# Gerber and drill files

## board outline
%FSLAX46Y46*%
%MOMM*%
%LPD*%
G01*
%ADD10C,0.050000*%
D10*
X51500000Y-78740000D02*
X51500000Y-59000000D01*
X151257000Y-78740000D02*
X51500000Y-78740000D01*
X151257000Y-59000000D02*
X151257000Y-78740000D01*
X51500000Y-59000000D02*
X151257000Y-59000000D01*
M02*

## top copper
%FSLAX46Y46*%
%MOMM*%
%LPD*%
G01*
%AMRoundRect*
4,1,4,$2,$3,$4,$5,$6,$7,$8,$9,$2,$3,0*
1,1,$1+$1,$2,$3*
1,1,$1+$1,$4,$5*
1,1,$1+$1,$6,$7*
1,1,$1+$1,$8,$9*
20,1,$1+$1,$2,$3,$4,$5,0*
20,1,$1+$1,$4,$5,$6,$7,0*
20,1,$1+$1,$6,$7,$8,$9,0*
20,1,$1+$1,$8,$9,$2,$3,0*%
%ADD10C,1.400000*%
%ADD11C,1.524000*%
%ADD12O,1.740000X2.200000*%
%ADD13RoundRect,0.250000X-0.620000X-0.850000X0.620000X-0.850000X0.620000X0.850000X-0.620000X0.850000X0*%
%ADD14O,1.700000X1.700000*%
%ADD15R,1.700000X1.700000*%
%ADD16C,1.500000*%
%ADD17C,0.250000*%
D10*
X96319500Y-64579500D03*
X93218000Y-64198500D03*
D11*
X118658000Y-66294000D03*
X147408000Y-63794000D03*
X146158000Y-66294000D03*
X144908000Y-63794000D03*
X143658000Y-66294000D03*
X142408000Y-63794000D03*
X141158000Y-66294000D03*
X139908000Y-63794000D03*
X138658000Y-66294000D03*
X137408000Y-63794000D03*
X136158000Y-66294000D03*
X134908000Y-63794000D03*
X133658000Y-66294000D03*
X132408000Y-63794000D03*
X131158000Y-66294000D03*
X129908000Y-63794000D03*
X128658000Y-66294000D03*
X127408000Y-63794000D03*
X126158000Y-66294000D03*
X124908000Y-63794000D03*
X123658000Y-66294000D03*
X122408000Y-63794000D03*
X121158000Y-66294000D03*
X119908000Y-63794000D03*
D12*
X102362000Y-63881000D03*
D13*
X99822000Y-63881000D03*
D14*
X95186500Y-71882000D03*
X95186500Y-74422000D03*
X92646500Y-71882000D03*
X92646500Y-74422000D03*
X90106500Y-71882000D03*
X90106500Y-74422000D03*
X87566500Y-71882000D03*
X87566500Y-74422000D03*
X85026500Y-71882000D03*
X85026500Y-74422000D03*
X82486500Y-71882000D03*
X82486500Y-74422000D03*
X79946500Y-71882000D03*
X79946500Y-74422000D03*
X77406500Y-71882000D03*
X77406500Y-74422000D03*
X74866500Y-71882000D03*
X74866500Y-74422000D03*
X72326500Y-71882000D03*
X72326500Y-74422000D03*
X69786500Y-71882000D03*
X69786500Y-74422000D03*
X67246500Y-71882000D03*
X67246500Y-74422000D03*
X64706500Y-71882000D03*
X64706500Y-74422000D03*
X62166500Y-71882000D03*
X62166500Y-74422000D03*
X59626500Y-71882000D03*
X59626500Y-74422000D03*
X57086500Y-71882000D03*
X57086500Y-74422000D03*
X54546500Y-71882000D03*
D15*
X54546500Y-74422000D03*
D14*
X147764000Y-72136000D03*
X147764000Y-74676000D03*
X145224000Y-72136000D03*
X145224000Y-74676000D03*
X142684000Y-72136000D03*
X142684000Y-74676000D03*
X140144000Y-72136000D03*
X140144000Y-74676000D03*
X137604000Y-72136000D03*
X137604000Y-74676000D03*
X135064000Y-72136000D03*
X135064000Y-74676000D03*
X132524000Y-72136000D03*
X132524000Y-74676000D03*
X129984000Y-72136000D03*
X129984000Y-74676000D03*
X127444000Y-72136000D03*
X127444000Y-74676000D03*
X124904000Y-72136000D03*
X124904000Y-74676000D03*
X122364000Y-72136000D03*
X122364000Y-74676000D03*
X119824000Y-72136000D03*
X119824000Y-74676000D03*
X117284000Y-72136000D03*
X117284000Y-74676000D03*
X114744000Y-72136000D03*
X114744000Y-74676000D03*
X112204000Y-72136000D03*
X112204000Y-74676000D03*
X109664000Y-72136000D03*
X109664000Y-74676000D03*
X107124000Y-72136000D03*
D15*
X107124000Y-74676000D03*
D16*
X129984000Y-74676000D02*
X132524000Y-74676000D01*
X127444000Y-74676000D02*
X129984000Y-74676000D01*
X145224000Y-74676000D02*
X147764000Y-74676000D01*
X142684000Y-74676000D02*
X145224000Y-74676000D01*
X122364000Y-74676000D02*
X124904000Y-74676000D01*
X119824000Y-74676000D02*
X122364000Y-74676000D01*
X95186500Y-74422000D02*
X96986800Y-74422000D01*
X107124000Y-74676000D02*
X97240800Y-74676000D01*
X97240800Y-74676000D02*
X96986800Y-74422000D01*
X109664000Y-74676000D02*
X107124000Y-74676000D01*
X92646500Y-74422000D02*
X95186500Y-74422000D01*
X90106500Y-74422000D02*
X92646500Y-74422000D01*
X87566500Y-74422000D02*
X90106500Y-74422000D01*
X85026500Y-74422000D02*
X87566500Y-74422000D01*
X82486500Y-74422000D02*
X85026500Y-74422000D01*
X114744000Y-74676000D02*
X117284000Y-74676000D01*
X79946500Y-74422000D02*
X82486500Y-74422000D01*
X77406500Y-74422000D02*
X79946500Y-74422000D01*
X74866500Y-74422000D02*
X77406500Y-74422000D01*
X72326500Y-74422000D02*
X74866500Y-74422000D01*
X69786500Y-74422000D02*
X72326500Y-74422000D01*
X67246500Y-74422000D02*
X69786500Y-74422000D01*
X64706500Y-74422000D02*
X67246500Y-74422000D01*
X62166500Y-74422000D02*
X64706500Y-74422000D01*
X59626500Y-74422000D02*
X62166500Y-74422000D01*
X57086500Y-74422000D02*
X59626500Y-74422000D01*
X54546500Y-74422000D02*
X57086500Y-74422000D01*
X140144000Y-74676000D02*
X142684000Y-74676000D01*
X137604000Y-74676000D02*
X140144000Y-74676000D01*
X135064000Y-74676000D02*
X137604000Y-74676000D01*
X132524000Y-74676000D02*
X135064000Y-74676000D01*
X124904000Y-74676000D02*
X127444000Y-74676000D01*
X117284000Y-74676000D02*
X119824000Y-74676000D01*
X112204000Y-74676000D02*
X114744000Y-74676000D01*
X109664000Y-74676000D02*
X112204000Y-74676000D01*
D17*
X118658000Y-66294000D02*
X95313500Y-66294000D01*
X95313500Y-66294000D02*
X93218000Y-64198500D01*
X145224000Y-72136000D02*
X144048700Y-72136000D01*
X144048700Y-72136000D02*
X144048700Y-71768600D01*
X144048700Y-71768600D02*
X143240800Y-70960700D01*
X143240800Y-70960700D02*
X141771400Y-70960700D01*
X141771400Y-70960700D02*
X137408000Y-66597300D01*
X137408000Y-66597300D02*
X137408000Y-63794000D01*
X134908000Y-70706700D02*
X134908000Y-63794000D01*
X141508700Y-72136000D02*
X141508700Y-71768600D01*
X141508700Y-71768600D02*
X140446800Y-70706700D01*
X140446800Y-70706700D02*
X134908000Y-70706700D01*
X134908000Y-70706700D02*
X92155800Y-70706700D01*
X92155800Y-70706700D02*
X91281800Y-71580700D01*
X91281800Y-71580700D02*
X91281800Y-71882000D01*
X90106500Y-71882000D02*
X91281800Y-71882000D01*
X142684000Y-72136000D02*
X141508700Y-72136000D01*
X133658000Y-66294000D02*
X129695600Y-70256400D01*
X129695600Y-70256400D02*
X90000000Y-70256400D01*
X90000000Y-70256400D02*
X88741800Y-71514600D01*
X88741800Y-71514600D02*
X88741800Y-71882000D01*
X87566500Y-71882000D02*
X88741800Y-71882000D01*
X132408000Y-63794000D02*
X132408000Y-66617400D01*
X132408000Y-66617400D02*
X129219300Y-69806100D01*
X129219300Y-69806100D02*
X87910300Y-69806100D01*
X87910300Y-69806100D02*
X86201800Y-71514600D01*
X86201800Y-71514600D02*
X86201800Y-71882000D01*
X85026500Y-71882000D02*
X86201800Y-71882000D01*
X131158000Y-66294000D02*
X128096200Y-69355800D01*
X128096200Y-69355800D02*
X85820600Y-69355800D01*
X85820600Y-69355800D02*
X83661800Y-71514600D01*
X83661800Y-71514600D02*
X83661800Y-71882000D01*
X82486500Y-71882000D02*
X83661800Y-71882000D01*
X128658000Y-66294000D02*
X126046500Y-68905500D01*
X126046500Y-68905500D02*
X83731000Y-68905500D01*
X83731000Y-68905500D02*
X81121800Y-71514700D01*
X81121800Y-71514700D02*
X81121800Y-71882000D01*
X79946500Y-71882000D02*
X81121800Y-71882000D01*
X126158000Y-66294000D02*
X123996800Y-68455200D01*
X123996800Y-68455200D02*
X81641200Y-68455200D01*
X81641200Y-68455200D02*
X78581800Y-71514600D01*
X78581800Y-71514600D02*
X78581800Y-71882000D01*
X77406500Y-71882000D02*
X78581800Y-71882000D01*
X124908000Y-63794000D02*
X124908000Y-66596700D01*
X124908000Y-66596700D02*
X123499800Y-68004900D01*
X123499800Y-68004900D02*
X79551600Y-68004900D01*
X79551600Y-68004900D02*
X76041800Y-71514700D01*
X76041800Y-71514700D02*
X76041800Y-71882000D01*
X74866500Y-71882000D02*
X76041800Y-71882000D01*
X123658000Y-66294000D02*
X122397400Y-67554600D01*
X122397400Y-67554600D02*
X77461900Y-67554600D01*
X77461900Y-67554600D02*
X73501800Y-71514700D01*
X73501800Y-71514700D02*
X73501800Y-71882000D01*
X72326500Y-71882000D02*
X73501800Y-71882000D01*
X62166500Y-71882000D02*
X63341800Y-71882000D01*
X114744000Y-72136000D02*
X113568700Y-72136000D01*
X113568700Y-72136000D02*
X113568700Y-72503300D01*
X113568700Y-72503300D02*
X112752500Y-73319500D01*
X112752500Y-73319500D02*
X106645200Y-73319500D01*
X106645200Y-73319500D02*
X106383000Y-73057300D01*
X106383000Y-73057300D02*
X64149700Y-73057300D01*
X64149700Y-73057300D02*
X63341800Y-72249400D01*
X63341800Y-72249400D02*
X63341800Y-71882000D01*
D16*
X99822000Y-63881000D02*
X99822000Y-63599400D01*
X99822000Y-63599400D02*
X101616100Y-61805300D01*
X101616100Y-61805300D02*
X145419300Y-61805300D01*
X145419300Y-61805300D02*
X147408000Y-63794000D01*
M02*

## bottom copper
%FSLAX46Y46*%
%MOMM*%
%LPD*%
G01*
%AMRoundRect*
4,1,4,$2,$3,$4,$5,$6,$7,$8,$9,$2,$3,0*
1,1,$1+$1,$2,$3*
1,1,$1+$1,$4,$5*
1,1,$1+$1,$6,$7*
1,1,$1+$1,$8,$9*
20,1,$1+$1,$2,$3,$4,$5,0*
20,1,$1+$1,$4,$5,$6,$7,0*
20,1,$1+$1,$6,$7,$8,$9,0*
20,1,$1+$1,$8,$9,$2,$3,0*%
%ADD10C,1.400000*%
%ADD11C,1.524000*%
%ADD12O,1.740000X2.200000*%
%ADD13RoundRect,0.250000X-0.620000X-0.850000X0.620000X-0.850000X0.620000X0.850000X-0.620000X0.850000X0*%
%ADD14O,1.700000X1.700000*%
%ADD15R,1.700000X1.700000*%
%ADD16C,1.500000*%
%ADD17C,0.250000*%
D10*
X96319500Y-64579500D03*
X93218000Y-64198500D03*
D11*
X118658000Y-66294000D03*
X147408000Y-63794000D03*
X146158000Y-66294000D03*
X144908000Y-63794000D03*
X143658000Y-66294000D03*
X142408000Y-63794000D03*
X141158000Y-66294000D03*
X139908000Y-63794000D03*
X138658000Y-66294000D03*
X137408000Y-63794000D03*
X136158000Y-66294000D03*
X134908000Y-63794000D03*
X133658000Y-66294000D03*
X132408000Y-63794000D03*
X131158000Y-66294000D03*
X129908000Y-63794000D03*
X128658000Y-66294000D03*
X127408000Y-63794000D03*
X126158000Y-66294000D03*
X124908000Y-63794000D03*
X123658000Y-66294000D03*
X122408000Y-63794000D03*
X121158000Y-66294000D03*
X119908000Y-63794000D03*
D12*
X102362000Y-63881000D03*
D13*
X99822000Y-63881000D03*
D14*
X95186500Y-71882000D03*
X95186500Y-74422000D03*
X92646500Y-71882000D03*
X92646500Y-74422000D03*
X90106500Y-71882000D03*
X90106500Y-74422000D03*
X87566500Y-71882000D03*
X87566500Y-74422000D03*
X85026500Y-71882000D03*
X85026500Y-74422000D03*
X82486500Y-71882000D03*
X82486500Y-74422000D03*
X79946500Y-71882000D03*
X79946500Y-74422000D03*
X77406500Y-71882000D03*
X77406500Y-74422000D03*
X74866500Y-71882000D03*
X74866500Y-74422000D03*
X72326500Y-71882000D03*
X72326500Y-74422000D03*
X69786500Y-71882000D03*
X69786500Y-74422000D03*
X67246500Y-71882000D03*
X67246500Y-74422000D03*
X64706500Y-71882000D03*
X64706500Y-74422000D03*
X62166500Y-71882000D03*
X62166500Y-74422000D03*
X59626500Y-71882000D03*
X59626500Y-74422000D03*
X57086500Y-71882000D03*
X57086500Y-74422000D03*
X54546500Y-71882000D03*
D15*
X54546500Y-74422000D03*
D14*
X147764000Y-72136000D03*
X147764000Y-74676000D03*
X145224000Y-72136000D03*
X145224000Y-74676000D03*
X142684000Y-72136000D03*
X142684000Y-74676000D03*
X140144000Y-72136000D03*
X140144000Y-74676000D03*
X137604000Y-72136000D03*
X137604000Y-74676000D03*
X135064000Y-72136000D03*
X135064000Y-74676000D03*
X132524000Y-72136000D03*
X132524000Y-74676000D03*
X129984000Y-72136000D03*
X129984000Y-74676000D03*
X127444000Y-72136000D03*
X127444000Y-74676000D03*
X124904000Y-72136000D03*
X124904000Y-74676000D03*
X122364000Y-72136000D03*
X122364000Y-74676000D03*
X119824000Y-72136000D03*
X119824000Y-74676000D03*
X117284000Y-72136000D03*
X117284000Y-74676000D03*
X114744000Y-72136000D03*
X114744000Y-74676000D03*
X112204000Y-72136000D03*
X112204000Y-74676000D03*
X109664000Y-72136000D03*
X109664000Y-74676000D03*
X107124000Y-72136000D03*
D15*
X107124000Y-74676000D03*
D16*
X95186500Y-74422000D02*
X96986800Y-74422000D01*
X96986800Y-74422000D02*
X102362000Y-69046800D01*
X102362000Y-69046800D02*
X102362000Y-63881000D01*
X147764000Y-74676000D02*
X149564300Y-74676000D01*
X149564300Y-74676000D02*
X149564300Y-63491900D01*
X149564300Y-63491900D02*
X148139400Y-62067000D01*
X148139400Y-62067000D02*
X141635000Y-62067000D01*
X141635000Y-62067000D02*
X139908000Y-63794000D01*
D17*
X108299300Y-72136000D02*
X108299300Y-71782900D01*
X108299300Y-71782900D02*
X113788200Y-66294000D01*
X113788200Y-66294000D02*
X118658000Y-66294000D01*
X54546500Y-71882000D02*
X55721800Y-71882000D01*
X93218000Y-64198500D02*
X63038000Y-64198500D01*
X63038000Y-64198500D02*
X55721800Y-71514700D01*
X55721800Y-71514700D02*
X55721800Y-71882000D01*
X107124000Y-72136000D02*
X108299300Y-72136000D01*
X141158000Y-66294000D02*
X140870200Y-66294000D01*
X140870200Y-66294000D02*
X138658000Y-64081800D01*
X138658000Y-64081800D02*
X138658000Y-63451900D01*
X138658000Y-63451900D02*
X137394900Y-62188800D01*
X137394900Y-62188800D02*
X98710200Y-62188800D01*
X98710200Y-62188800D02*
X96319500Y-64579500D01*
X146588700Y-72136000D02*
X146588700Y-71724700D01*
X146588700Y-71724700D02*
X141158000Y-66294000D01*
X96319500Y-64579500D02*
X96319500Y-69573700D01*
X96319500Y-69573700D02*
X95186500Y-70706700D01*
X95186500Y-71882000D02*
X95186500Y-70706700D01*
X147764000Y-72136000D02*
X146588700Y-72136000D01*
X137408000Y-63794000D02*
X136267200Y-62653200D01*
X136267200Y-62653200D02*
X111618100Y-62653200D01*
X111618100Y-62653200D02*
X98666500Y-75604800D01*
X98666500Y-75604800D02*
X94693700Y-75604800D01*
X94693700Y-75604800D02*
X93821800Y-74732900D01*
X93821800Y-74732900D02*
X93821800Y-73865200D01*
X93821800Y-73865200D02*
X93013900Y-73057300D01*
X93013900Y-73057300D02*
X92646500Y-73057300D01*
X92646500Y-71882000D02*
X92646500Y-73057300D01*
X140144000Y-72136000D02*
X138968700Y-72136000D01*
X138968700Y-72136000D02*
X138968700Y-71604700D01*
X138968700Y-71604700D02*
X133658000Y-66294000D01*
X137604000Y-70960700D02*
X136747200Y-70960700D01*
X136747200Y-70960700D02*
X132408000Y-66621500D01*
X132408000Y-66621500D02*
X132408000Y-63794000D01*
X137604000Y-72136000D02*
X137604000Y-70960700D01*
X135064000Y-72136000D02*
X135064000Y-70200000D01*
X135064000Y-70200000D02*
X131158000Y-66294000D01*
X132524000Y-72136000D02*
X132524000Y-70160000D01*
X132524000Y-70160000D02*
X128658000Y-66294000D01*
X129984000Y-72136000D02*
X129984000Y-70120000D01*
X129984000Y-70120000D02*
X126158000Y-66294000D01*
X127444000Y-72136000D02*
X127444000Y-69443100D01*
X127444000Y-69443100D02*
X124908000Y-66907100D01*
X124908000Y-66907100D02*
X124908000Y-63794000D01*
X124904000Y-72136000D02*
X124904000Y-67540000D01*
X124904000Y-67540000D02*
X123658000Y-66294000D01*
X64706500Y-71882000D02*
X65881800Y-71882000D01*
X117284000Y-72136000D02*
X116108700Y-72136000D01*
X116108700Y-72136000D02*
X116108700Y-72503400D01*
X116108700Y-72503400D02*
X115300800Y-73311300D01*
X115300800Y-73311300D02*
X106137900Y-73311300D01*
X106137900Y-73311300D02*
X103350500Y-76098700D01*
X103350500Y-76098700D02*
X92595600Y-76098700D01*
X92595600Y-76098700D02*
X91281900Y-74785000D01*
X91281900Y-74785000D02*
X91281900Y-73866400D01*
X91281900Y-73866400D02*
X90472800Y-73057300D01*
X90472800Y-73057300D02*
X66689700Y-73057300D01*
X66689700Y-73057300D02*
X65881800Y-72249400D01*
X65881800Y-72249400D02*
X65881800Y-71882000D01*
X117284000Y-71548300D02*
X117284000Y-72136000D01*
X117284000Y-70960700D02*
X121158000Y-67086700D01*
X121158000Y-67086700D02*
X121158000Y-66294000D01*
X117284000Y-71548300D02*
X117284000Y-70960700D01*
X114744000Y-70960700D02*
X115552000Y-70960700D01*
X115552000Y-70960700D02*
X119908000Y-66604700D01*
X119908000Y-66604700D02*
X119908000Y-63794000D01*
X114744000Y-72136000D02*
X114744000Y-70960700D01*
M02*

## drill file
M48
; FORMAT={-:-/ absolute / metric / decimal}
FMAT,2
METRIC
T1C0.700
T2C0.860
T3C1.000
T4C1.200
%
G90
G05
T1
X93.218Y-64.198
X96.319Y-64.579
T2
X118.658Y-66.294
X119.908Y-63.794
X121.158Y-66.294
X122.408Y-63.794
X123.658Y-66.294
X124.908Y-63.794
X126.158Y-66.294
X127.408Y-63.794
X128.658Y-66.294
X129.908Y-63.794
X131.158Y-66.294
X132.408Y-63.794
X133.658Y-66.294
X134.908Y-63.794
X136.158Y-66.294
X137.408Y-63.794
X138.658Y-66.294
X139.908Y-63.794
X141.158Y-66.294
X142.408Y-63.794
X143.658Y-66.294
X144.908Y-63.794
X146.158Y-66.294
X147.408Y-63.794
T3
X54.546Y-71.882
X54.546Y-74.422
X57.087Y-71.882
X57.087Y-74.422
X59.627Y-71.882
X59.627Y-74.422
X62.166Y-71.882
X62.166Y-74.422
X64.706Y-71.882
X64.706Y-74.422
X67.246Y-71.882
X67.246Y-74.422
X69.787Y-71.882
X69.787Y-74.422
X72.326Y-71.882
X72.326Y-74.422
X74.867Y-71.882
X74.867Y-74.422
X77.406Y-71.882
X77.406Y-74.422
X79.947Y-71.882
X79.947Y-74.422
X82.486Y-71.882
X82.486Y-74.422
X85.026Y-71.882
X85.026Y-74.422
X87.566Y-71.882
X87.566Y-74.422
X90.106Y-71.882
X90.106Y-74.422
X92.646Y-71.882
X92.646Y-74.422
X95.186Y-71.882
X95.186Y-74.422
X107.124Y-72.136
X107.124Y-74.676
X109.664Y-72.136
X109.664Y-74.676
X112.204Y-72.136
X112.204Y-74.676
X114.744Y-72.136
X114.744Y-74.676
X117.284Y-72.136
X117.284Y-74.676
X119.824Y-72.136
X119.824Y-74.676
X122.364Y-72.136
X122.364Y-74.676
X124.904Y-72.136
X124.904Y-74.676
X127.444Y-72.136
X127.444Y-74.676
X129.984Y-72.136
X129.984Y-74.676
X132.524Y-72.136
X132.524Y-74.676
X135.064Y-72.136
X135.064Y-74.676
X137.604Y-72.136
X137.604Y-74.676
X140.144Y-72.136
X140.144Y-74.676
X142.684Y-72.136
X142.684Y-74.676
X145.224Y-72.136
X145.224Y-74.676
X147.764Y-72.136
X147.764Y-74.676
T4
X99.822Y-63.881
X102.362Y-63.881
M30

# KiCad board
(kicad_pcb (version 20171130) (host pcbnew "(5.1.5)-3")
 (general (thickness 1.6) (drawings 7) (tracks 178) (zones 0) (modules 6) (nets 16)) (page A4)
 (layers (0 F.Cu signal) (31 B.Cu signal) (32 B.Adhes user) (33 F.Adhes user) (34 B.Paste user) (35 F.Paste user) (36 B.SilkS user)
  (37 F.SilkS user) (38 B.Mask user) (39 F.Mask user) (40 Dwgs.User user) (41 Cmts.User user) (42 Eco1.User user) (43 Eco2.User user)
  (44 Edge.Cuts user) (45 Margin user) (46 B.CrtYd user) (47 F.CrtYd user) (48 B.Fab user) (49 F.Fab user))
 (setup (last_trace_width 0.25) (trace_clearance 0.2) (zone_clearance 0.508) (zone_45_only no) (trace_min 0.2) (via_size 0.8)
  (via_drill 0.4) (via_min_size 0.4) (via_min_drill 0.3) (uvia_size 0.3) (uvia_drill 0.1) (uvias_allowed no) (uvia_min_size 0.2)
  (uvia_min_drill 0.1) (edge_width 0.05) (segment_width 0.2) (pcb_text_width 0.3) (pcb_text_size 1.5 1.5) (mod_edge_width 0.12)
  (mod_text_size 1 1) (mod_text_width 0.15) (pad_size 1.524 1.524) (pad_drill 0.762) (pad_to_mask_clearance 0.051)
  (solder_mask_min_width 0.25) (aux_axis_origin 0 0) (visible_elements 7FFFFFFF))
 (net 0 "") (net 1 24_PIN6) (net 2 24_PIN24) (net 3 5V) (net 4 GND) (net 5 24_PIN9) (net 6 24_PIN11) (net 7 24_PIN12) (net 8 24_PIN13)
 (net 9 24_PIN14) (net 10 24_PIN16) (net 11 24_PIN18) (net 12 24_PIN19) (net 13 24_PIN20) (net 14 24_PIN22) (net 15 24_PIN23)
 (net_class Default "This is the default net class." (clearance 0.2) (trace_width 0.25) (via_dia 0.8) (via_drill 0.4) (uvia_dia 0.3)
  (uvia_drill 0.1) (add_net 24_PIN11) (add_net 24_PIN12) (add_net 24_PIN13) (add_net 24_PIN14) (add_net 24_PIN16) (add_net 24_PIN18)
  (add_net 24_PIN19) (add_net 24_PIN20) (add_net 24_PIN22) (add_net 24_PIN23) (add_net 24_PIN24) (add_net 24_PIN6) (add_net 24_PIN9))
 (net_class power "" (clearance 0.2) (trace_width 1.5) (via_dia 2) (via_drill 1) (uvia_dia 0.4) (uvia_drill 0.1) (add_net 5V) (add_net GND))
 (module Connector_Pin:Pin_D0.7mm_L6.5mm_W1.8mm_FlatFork (layer F.Cu) (at 96.3195 64.5795)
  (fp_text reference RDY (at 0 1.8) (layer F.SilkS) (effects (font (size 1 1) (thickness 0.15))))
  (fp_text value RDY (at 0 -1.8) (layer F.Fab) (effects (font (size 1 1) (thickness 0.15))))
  (pad 1 thru_hole circle (at 0 0) (size 1.4 1.4) (drill 0.7) (layers *.Cu *.Mask) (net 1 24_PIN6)))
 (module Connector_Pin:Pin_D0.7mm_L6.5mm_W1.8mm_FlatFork (layer F.Cu) (at 93.218 64.1985)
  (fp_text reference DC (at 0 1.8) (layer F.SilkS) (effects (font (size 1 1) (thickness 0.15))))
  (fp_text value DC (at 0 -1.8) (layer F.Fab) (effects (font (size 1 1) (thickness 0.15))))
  (pad 1 thru_hole circle (at 0 0) (size 1.4 1.4) (drill 0.7) (layers *.Cu *.Mask) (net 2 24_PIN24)))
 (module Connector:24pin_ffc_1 (layer F.Cu) (at 121.158 66.294)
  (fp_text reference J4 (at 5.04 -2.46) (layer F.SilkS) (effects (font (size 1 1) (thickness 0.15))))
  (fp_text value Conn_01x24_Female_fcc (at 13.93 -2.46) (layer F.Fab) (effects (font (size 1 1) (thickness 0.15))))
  (pad 24 thru_hole circle (at -2.5 0) (size 1.524 1.524) (drill 0.86) (layers *.Cu *.Mask) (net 2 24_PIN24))
  (pad 1 thru_hole circle (at 26.25 -2.5) (size 1.524 1.524) (drill 0.86) (layers *.Cu *.Mask) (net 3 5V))
  (pad 2 thru_hole circle (at 25 0) (size 1.524 1.524) (drill 0.86) (layers *.Cu *.Mask))
  (pad 3 thru_hole circle (at 23.75 -2.5) (size 1.524 1.524) (drill 0.86) (layers *.Cu *.Mask))
  (pad 4 thru_hole circle (at 22.5 0) (size 1.524 1.524) (drill 0.86) (layers *.Cu *.Mask))
  (pad 5 thru_hole circle (at 21.25 -2.5) (size 1.524 1.524) (drill 0.86) (layers *.Cu *.Mask))
  (pad 6 thru_hole circle (at 20 0) (size 1.524 1.524) (drill 0.86) (layers *.Cu *.Mask) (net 1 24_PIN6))
  (pad 7 thru_hole circle (at 18.75 -2.5) (size 1.524 1.524) (drill 0.86) (layers *.Cu *.Mask) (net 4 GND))
  (pad 8 thru_hole circle (at 17.5 0) (size 1.524 1.524) (drill 0.86) (layers *.Cu *.Mask))
  (pad 9 thru_hole circle (at 16.25 -2.5) (size 1.524 1.524) (drill 0.86) (layers *.Cu *.Mask) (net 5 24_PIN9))
  (pad 10 thru_hole circle (at 15 0) (size 1.524 1.524) (drill 0.86) (layers *.Cu *.Mask))
  (pad 11 thru_hole circle (at 13.75 -2.5) (size 1.524 1.524) (drill 0.86) (layers *.Cu *.Mask) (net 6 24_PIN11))
  (pad 12 thru_hole circle (at 12.5 0) (size 1.524 1.524) (drill 0.86) (layers *.Cu *.Mask) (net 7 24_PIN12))
  (pad 13 thru_hole circle (at 11.25 -2.5) (size 1.524 1.524) (drill 0.86) (layers *.Cu *.Mask) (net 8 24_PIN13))
  (pad 14 thru_hole circle (at 10 0) (size 1.524 1.524) (drill 0.86) (layers *.Cu *.Mask) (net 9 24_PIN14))
  (pad 15 thru_hole circle (at 8.75 -2.5) (size 1.524 1.524) (drill 0.86) (layers *.Cu *.Mask))
  (pad 16 thru_hole circle (at 7.5 0) (size 1.524 1.524) (drill 0.86) (layers *.Cu *.Mask) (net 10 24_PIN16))
  (pad 17 thru_hole circle (at 6.25 -2.5) (size 1.524 1.524) (drill 0.86) (layers *.Cu *.Mask))
  (pad 18 thru_hole circle (at 5 0) (size 1.524 1.524) (drill 0.86) (layers *.Cu *.Mask) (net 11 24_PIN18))
  (pad 19 thru_hole circle (at 3.75 -2.5) (size 1.524 1.524) (drill 0.86) (layers *.Cu *.Mask) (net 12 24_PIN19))
  (pad 20 thru_hole circle (at 2.5 0) (size 1.524 1.524) (drill 0.86) (layers *.Cu *.Mask) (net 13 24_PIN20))
  (pad 21 thru_hole circle (at 1.25 -2.5) (size 1.524 1.524) (drill 0.86) (layers *.Cu *.Mask))
  (pad 22 thru_hole circle (at 0 0) (size 1.524 1.524) (drill 0.86) (layers *.Cu *.Mask) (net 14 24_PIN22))
  (pad 23 thru_hole circle (at -1.25 -2.5) (size 1.524 1.524) (drill 0.86) (layers *.Cu *.Mask) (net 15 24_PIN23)))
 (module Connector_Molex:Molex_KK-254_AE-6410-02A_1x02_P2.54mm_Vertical (layer F.Cu) (at 99.822 63.881)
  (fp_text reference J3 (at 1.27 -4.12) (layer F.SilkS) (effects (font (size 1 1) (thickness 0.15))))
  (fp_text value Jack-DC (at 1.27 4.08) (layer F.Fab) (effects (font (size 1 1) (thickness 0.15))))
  (pad 2 thru_hole oval (at 2.54 0) (size 1.74 2.2) (drill 1.2) (layers *.Cu *.Mask) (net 4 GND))
  (pad 1 thru_hole roundrect (at 0 0) (size 1.74 2.2) (drill 1.2) (layers *.Cu *.Mask) (roundrect_rratio 0.143678) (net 3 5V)))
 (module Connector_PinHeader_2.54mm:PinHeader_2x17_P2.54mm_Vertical (layer F.Cu) (at 54.5465 74.422 90)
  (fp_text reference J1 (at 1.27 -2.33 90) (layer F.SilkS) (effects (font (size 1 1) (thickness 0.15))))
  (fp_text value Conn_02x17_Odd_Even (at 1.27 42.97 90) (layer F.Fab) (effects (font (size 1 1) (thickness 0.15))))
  (pad 34 thru_hole oval (at 2.54 40.64 90) (size 1.7 1.7) (drill 1) (layers *.Cu *.Mask) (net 1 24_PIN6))
  (pad 33 thru_hole oval (at 0 40.64 90) (size 1.7 1.7) (drill 1) (layers *.Cu *.Mask) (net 4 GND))
  (pad 32 thru_hole oval (at 2.54 38.1 90) (size 1.7 1.7) (drill 1) (layers *.Cu *.Mask) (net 5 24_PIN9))
  (pad 31 thru_hole oval (at 0 38.1 90) (size 1.7 1.7) (drill 1) (layers *.Cu *.Mask) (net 4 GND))
  (pad 30 thru_hole oval (at 2.54 35.56 90) (size 1.7 1.7) (drill 1) (layers *.Cu *.Mask) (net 6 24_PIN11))
  (pad 29 thru_hole oval (at 0 35.56 90) (size 1.7 1.7) (drill 1) (layers *.Cu *.Mask) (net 4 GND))
  (pad 28 thru_hole oval (at 2.54 33.02 90) (size 1.7 1.7) (drill 1) (layers *.Cu *.Mask) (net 7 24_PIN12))
  (pad 27 thru_hole oval (at 0 33.02 90) (size 1.7 1.7) (drill 1) (layers *.Cu *.Mask) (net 4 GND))
  (pad 26 thru_hole oval (at 2.54 30.48 90) (size 1.7 1.7) (drill 1) (layers *.Cu *.Mask) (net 8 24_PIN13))
  (pad 25 thru_hole oval (at 0 30.48 90) (size 1.7 1.7) (drill 1) (layers *.Cu *.Mask) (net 4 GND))
  (pad 24 thru_hole oval (at 2.54 27.94 90) (size 1.7 1.7) (drill 1) (layers *.Cu *.Mask) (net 9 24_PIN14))
  (pad 23 thru_hole oval (at 0 27.94 90) (size 1.7 1.7) (drill 1) (layers *.Cu *.Mask) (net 4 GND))
  (pad 22 thru_hole oval (at 2.54 25.4 90) (size 1.7 1.7) (drill 1) (layers *.Cu *.Mask) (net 10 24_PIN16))
  (pad 21 thru_hole oval (at 0 25.4 90) (size 1.7 1.7) (drill 1) (layers *.Cu *.Mask) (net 4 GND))
  (pad 20 thru_hole oval (at 2.54 22.86 90) (size 1.7 1.7) (drill 1) (layers *.Cu *.Mask) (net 11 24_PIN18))
  (pad 19 thru_hole oval (at 0 22.86 90) (size 1.7 1.7) (drill 1) (layers *.Cu *.Mask) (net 4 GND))
  (pad 18 thru_hole oval (at 2.54 20.32 90) (size 1.7 1.7) (drill 1) (layers *.Cu *.Mask) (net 12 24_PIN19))
  (pad 17 thru_hole oval (at 0 20.32 90) (size 1.7 1.7) (drill 1) (layers *.Cu *.Mask) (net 4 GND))
  (pad 16 thru_hole oval (at 2.54 17.78 90) (size 1.7 1.7) (drill 1) (layers *.Cu *.Mask) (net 13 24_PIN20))
  (pad 15 thru_hole oval (at 0 17.78 90) (size 1.7 1.7) (drill 1) (layers *.Cu *.Mask) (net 4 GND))
  (pad 14 thru_hole oval (at 2.54 15.24 90) (size 1.7 1.7) (drill 1) (layers *.Cu *.Mask))
  (pad 13 thru_hole oval (at 0 15.24 90) (size 1.7 1.7) (drill 1) (layers *.Cu *.Mask) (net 4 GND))
  (pad 12 thru_hole oval (at 2.54 12.7 90) (size 1.7 1.7) (drill 1) (layers *.Cu *.Mask))
  (pad 11 thru_hole oval (at 0 12.7 90) (size 1.7 1.7) (drill 1) (layers *.Cu *.Mask) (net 4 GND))
  (pad 10 thru_hole oval (at 2.54 10.16 90) (size 1.7 1.7) (drill 1) (layers *.Cu *.Mask) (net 14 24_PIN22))
  (pad 9 thru_hole oval (at 0 10.16 90) (size 1.7 1.7) (drill 1) (layers *.Cu *.Mask) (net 4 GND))
  (pad 8 thru_hole oval (at 2.54 7.62 90) (size 1.7 1.7) (drill 1) (layers *.Cu *.Mask) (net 15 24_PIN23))
  (pad 7 thru_hole oval (at 0 7.62 90) (size 1.7 1.7) (drill 1) (layers *.Cu *.Mask) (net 4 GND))
  (pad 6 thru_hole oval (at 2.54 5.08 90) (size 1.7 1.7) (drill 1) (layers *.Cu *.Mask))
  (pad 5 thru_hole oval (at 0 5.08 90) (size 1.7 1.7) (drill 1) (layers *.Cu *.Mask) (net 4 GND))
  (pad 4 thru_hole oval (at 2.54 2.54 90) (size 1.7 1.7) (drill 1) (layers *.Cu *.Mask))
  (pad 3 thru_hole oval (at 0 2.54 90) (size 1.7 1.7) (drill 1) (layers *.Cu *.Mask) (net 4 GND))
  (pad 2 thru_hole oval (at 2.54 0 90) (size 1.7 1.7) (drill 1) (layers *.Cu *.Mask) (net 2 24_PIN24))
  (pad 1 thru_hole rect (at 0 0 90) (size 1.7 1.7) (drill 1) (layers *.Cu *.Mask) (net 4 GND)))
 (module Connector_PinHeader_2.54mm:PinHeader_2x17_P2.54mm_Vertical (layer F.Cu) (at 107.124 74.676 90)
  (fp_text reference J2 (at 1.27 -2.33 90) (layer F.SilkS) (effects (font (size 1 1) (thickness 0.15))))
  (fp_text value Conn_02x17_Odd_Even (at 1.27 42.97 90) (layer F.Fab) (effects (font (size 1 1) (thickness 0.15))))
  (pad 34 thru_hole oval (at 2.54 40.64 90) (size 1.7 1.7) (drill 1) (layers *.Cu *.Mask) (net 1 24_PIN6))
  (pad 33 thru_hole oval (at 0 40.64 90) (size 1.7 1.7) (drill 1) (layers *.Cu *.Mask) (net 4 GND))
  (pad 32 thru_hole oval (at 2.54 38.1 90) (size 1.7 1.7) (drill 1) (layers *.Cu *.Mask) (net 5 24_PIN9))
  (pad 31 thru_hole oval (at 0 38.1 90) (size 1.7 1.7) (drill 1) (layers *.Cu *.Mask) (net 4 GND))
  (pad 30 thru_hole oval (at 2.54 35.56 90) (size 1.7 1.7) (drill 1) (layers *.Cu *.Mask) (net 6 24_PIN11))
  (pad 29 thru_hole oval (at 0 35.56 90) (size 1.7 1.7) (drill 1) (layers *.Cu *.Mask) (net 4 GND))
  (pad 28 thru_hole oval (at 2.54 33.02 90) (size 1.7 1.7) (drill 1) (layers *.Cu *.Mask) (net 7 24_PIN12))
  (pad 27 thru_hole oval (at 0 33.02 90) (size 1.7 1.7) (drill 1) (layers *.Cu *.Mask) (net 4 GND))
  (pad 26 thru_hole oval (at 2.54 30.48 90) (size 1.7 1.7) (drill 1) (layers *.Cu *.Mask) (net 8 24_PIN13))
  (pad 25 thru_hole oval (at 0 30.48 90) (size 1.7 1.7) (drill 1) (layers *.Cu *.Mask) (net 4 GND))
  (pad 24 thru_hole oval (at 2.54 27.94 90) (size 1.7 1.7) (drill 1) (layers *.Cu *.Mask) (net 9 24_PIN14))
  (pad 23 thru_hole oval (at 0 27.94 90) (size 1.7 1.7) (drill 1) (layers *.Cu *.Mask) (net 4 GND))
  (pad 22 thru_hole oval (at 2.54 25.4 90) (size 1.7 1.7) (drill 1) (layers *.Cu *.Mask) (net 10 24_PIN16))
  (pad 21 thru_hole oval (at 0 25.4 90) (size 1.7 1.7) (drill 1) (layers *.Cu *.Mask) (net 4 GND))
  (pad 20 thru_hole oval (at 2.54 22.86 90) (size 1.7 1.7) (drill 1) (layers *.Cu *.Mask) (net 11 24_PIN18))
  (pad 19 thru_hole oval (at 0 22.86 90) (size 1.7 1.7) (drill 1) (layers *.Cu *.Mask) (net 4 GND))
  (pad 18 thru_hole oval (at 2.54 20.32 90) (size 1.7 1.7) (drill 1) (layers *.Cu *.Mask) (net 12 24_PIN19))
  (pad 17 thru_hole oval (at 0 20.32 90) (size 1.7 1.7) (drill 1) (layers *.Cu *.Mask) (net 4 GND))
  (pad 16 thru_hole oval (at 2.54 17.78 90) (size 1.7 1.7) (drill 1) (layers *.Cu *.Mask) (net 13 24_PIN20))
  (pad 15 thru_hole oval (at 0 17.78 90) (size 1.7 1.7) (drill 1) (layers *.Cu *.Mask) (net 4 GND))
  (pad 14 thru_hole oval (at 2.54 15.24 90) (size 1.7 1.7) (drill 1) (layers *.Cu *.Mask))
  (pad 13 thru_hole oval (at 0 15.24 90) (size 1.7 1.7) (drill 1) (layers *.Cu *.Mask) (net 4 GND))
  (pad 12 thru_hole oval (at 2.54 12.7 90) (size 1.7 1.7) (drill 1) (layers *.Cu *.Mask))
  (pad 11 thru_hole oval (at 0 12.7 90) (size 1.7 1.7) (drill 1) (layers *.Cu *.Mask) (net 4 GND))
  (pad 10 thru_hole oval (at 2.54 10.16 90) (size 1.7 1.7) (drill 1) (layers *.Cu *.Mask) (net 14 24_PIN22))
  (pad 9 thru_hole oval (at 0 10.16 90) (size 1.7 1.7) (drill 1) (layers *.Cu *.Mask) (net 4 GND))
  (pad 8 thru_hole oval (at 2.54 7.62 90) (size 1.7 1.7) (drill 1) (layers *.Cu *.Mask) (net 15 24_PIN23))
  (pad 7 thru_hole oval (at 0 7.62 90) (size 1.7 1.7) (drill 1) (layers *.Cu *.Mask) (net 4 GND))
  (pad 6 thru_hole oval (at 2.54 5.08 90) (size 1.7 1.7) (drill 1) (layers *.Cu *.Mask))
  (pad 5 thru_hole oval (at 0 5.08 90) (size 1.7 1.7) (drill 1) (layers *.Cu *.Mask) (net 4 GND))
  (pad 4 thru_hole oval (at 2.54 2.54 90) (size 1.7 1.7) (drill 1) (layers *.Cu *.Mask))
  (pad 3 thru_hole oval (at 0 2.54 90) (size 1.7 1.7) (drill 1) (layers *.Cu *.Mask) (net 4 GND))
  (pad 2 thru_hole oval (at 2.54 0 90) (size 1.7 1.7) (drill 1) (layers *.Cu *.Mask) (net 2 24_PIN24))
  (pad 1 thru_hole rect (at 0 0 90) (size 1.7 1.7) (drill 1) (layers *.Cu *.Mask) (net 4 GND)))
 (gr_line (start 51.5 78.74) (end 51.5 59) (layer Edge.Cuts) (width 0.05))
 (gr_line (start 151.257 78.74) (end 51.5 78.74) (layer Edge.Cuts) (width 0.05))
 (gr_line (start 151.257 59) (end 151.257 78.74) (layer Edge.Cuts) (width 0.05))
 (gr_line (start 51.5 59) (end 151.257 59) (layer Edge.Cuts) (width 0.05))
 (segment (start 129.984 74.676) (end 132.524 74.676) (width 1.5) (layer F.Cu) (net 4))
 (segment (start 127.444 74.676) (end 129.984 74.676) (width 1.5) (layer F.Cu) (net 4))
 (segment (start 145.224 74.676) (end 147.764 74.676) (width 1.5) (layer F.Cu) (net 4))
 (segment (start 142.684 74.676) (end 145.224 74.676) (width 1.5) (layer F.Cu) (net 4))
 (segment (start 95.1865 74.422) (end 96.9868 74.422) (width 1.5) (layer B.Cu) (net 4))
 (segment (start 96.9868 74.422) (end 102.362 69.0468) (width 1.5) (layer B.Cu) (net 4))
 (segment (start 102.362 69.0468) (end 102.362 63.881) (width 1.5) (layer B.Cu) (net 4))
 (segment (start 122.364 74.676) (end 124.904 74.676) (width 1.5) (layer F.Cu) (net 4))
 (segment (start 119.824 74.676) (end 122.364 74.676) (width 1.5) (layer F.Cu) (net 4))
 (segment (start 95.1865 74.422) (end 96.9868 74.422) (width 1.5) (layer F.Cu) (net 4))
 (segment (start 107.124 74.676) (end 97.2408 74.676) (width 1.5) (layer F.Cu) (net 4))
 (segment (start 97.2408 74.676) (end 96.9868 74.422) (width 1.5) (layer F.Cu) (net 4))
 (segment (start 109.664 74.676) (end 107.124 74.676) (width 1.5) (layer F.Cu) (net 4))
 (segment (start 147.764 74.676) (end 149.5643 74.676) (width 1.5) (layer B.Cu) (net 4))
 (segment (start 149.5643 74.676) (end 149.5643 63.4919) (width 1.5) (layer B.Cu) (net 4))
 (segment (start 149.5643 63.4919) (end 148.1394 62.067) (width 1.5) (layer B.Cu) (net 4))
 (segment (start 148.1394 62.067) (end 141.635 62.067) (width 1.5) (layer B.Cu) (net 4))
 (segment (start 141.635 62.067) (end 139.908 63.794) (width 1.5) (layer B.Cu) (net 4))
 (segment (start 92.6465 74.422) (end 95.1865 74.422) (width 1.5) (layer F.Cu) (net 4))
 (segment (start 90.1065 74.422) (end 92.6465 74.422) (width 1.5) (layer F.Cu) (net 4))
 (segment (start 87.5665 74.422) (end 90.1065 74.422) (width 1.5) (layer F.Cu) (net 4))
 (segment (start 85.0265 74.422) (end 87.5665 74.422) (width 1.5) (layer F.Cu) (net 4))
 (segment (start 82.4865 74.422) (end 85.0265 74.422) (width 1.5) (layer F.Cu) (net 4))
 (segment (start 114.744 74.676) (end 117.284 74.676) (width 1.5) (layer F.Cu) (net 4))
 (segment (start 79.9465 74.422) (end 82.4865 74.422) (width 1.5) (layer F.Cu) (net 4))
 (segment (start 77.4065 74.422) (end 79.9465 74.422) (width 1.5) (layer F.Cu) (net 4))
 (segment (start 74.8665 74.422) (end 77.4065 74.422) (width 1.5) (layer F.Cu) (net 4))
 (segment (start 72.3265 74.422) (end 74.8665 74.422) (width 1.5) (layer F.Cu) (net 4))
 (segment (start 69.7865 74.422) (end 72.3265 74.422) (width 1.5) (layer F.Cu) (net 4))
 (segment (start 67.2465 74.422) (end 69.7865 74.422) (width 1.5) (layer F.Cu) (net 4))
 (segment (start 64.7065 74.422) (end 67.2465 74.422) (width 1.5) (layer F.Cu) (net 4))
 (segment (start 62.1665 74.422) (end 64.7065 74.422) (width 1.5) (layer F.Cu) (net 4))
 (segment (start 59.6265 74.422) (end 62.1665 74.422) (width 1.5) (layer F.Cu) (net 4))
 (segment (start 57.0865 74.422) (end 59.6265 74.422) (width 1.5) (layer F.Cu) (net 4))
 (segment (start 54.5465 74.422) (end 57.0865 74.422) (width 1.5) (layer F.Cu) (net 4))
 (segment (start 140.144 74.676) (end 142.684 74.676) (width 1.5) (layer F.Cu) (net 4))
 (segment (start 137.604 74.676) (end 140.144 74.676) (width 1.5) (layer F.Cu) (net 4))
 (segment (start 135.064 74.676) (end 137.604 74.676) (width 1.5) (layer F.Cu) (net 4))
 (segment (start 132.524 74.676) (end 135.064 74.676) (width 1.5) (layer F.Cu) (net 4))
 (segment (start 124.904 74.676) (end 127.444 74.676) (width 1.5) (layer F.Cu) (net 4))
 (segment (start 117.284 74.676) (end 119.824 74.676) (width 1.5) (layer F.Cu) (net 4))
 (segment (start 112.204 74.676) (end 114.744 74.676) (width 1.5) (layer F.Cu) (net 4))
 (segment (start 109.664 74.676) (end 112.204 74.676) (width 1.5) (layer F.Cu) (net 4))
 (segment (start 108.2993 72.136) (end 108.2993 71.7829) (width 0.25) (layer B.Cu) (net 2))
 (segment (start 108.2993 71.7829) (end 113.7882 66.294) (width 0.25) (layer B.Cu) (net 2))
 (segment (start 113.7882 66.294) (end 118.658 66.294) (width 0.25) (layer B.Cu) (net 2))
 (segment (start 54.5465 71.882) (end 55.7218 71.882) (width 0.25) (layer B.Cu) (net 2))
 (segment (start 93.218 64.1985) (end 63.038 64.1985) (width 0.25) (layer B.Cu) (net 2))
 (segment (start 63.038 64.1985) (end 55.7218 71.5147) (width 0.25) (layer B.Cu) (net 2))
 (segment (start 55.7218 71.5147) (end 55.7218 71.882) (width 0.25) (layer B.Cu) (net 2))
 (segment (start 118.658 66.294) (end 95.3135 66.294) (width 0.25) (layer F.Cu) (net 2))
 (segment (start 95.3135 66.294) (end 93.218 64.1985) (width 0.25) (layer F.Cu) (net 2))
 (segment (start 107.124 72.136) (end 108.2993 72.136) (width 0.25) (layer B.Cu) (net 2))
 (segment (start 141.158 66.294) (end 140.8702 66.294) (width 0.25) (layer B.Cu) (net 1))
 (segment (start 140.8702 66.294) (end 138.658 64.0818) (width 0.25) (layer B.Cu) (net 1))
 (segment (start 138.658 64.0818) (end 138.658 63.4519) (width 0.25) (layer B.Cu) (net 1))
 (segment (start 138.658 63.4519) (end 137.3949 62.1888) (width 0.25) (layer B.Cu) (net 1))
 (segment (start 137.3949 62.1888) (end 98.7102 62.1888) (width 0.25) (layer B.Cu) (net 1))
 (segment (start 98.7102 62.1888) (end 96.3195 64.5795) (width 0.25) (layer B.Cu) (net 1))
 (segment (start 146.5887 72.136) (end 146.5887 71.7247) (width 0.25) (layer B.Cu) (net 1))
 (segment (start 146.5887 71.7247) (end 141.158 66.294) (width 0.25) (layer B.Cu) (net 1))
 (segment (start 96.3195 64.5795) (end 96.3195 69.5737) (width 0.25) (layer B.Cu) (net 1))
 (segment (start 96.3195 69.5737) (end 95.1865 70.7067) (width 0.25) (layer B.Cu) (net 1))
 (segment (start 95.1865 71.882) (end 95.1865 70.7067) (width 0.25) (layer B.Cu) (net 1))
 (segment (start 147.764 72.136) (end 146.5887 72.136) (width 0.25) (layer B.Cu) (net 1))
 (segment (start 137.408 63.794) (end 136.2672 62.6532) (width 0.25) (layer B.Cu) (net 5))
 (segment (start 136.2672 62.6532) (end 111.6181 62.6532) (width 0.25) (layer B.Cu) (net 5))
 (segment (start 111.6181 62.6532) (end 98.6665 75.6048) (width 0.25) (layer B.Cu) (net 5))
 (segment (start 98.6665 75.6048) (end 94.6937 75.6048) (width 0.25) (layer B.Cu) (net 5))
 (segment (start 94.6937 75.6048) (end 93.8218 74.7329) (width 0.25) (layer B.Cu) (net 5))
 (segment (start 93.8218 74.7329) (end 93.8218 73.8652) (width 0.25) (layer B.Cu) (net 5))
 (segment (start 93.8218 73.8652) (end 93.0139 73.0573) (width 0.25) (layer B.Cu) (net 5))
 (segment (start 93.0139 73.0573) (end 92.6465 73.0573) (width 0.25) (layer B.Cu) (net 5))
 (segment (start 92.6465 71.882) (end 92.6465 73.0573) (width 0.25) (layer B.Cu) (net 5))
 (segment (start 145.224 72.136) (end 144.0487 72.136) (width 0.25) (layer F.Cu) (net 5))
 (segment (start 144.0487 72.136) (end 144.0487 71.7686) (width 0.25) (layer F.Cu) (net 5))
 (segment (start 144.0487 71.7686) (end 143.2408 70.9607) (width 0.25) (layer F.Cu) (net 5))
 (segment (start 143.2408 70.9607) (end 141.7714 70.9607) (width 0.25) (layer F.Cu) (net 5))
 (segment (start 141.7714 70.9607) (end 137.408 66.5973) (width 0.25) (layer F.Cu) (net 5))
 (segment (start 137.408 66.5973) (end 137.408 63.794) (width 0.25) (layer F.Cu) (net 5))
 (segment (start 134.908 70.7067) (end 134.908 63.794) (width 0.25) (layer F.Cu) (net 6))
 (segment (start 141.5087 72.136) (end 141.5087 71.7686) (width 0.25) (layer F.Cu) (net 6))
 (segment (start 141.5087 71.7686) (end 140.4468 70.7067) (width 0.25) (layer F.Cu) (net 6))
 (segment (start 140.4468 70.7067) (end 134.908 70.7067) (width 0.25) (layer F.Cu) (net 6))
 (segment (start 134.908 70.7067) (end 92.1558 70.7067) (width 0.25) (layer F.Cu) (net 6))
 (segment (start 92.1558 70.7067) (end 91.2818 71.5807) (width 0.25) (layer F.Cu) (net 6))
 (segment (start 91.2818 71.5807) (end 91.2818 71.882) (width 0.25) (layer F.Cu) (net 6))
 (segment (start 90.1065 71.882) (end 91.2818 71.882) (width 0.25) (layer F.Cu) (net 6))
 (segment (start 142.684 72.136) (end 141.5087 72.136) (width 0.25) (layer F.Cu) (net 6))
 (segment (start 133.658 66.294) (end 129.6956 70.2564) (width 0.25) (layer F.Cu) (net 7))
 (segment (start 129.6956 70.2564) (end 90 70.2564) (width 0.25) (layer F.Cu) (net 7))
 (segment (start 90 70.2564) (end 88.7418 71.5146) (width 0.25) (layer F.Cu) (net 7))
 (segment (start 88.7418 71.5146) (end 88.7418 71.882) (width 0.25) (layer F.Cu) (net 7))
 (segment (start 87.5665 71.882) (end 88.7418 71.882) (width 0.25) (layer F.Cu) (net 7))
 (segment (start 140.144 72.136) (end 138.9687 72.136) (width 0.25) (layer B.Cu) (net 7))
 (segment (start 138.9687 72.136) (end 138.9687 71.6047) (width 0.25) (layer B.Cu) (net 7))
 (segment (start 138.9687 71.6047) (end 133.658 66.294) (width 0.25) (layer B.Cu) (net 7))
 (segment (start 132.408 63.794) (end 132.408 66.6174) (width 0.25) (layer F.Cu) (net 8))
 (segment (start 132.408 66.6174) (end 129.2193 69.8061) (width 0.25) (layer F.Cu) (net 8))
 (segment (start 129.2193 69.8061) (end 87.9103 69.8061) (width 0.25) (layer F.Cu) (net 8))
 (segment (start 87.9103 69.8061) (end 86.2018 71.5146) (width 0.25) (layer F.Cu) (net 8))
 (segment (start 86.2018 71.5146) (end 86.2018 71.882) (width 0.25) (layer F.Cu) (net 8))
 (segment (start 85.0265 71.882) (end 86.2018 71.882) (width 0.25) (layer F.Cu) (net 8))
 (segment (start 137.604 70.9607) (end 136.7472 70.9607) (width 0.25) (layer B.Cu) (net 8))
 (segment (start 136.7472 70.9607) (end 132.408 66.6215) (width 0.25) (layer B.Cu) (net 8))
 (segment (start 132.408 66.6215) (end 132.408 63.794) (width 0.25) (layer B.Cu) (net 8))
 (segment (start 137.604 72.136) (end 137.604 70.9607) (width 0.25) (layer B.Cu) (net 8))
 (segment (start 131.158 66.294) (end 128.0962 69.3558) (width 0.25) (layer F.Cu) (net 9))
 (segment (start 128.0962 69.3558) (end 85.8206 69.3558) (width 0.25) (layer F.Cu) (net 9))
 (segment (start 85.8206 69.3558) (end 83.6618 71.5146) (width 0.25) (layer F.Cu) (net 9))
 (segment (start 83.6618 71.5146) (end 83.6618 71.882) (width 0.25) (layer F.Cu) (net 9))
 (segment (start 82.4865 71.882) (end 83.6618 71.882) (width 0.25) (layer F.Cu) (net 9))
 (segment (start 135.064 72.136) (end 135.064 70.2) (width 0.25) (layer B.Cu) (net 9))
 (segment (start 135.064 70.2) (end 131.158 66.294) (width 0.25) (layer B.Cu) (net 9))
 (segment (start 128.658 66.294) (end 126.0465 68.9055) (width 0.25) (layer F.Cu) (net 10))
 (segment (start 126.0465 68.9055) (end 83.731 68.9055) (width 0.25) (layer F.Cu) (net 10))
 (segment (start 83.731 68.9055) (end 81.1218 71.5147) (width 0.25) (layer F.Cu) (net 10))
 (segment (start 81.1218 71.5147) (end 81.1218 71.882) (width 0.25) (layer F.Cu) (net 10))
 (segment (start 79.9465 71.882) (end 81.1218 71.882) (width 0.25) (layer F.Cu) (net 10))
 (segment (start 132.524 72.136) (end 132.524 70.16) (width 0.25) (layer B.Cu) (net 10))
 (segment (start 132.524 70.16) (end 128.658 66.294) (width 0.25) (layer B.Cu) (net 10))
 (segment (start 126.158 66.294) (end 123.9968 68.4552) (width 0.25) (layer F.Cu) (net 11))
 (segment (start 123.9968 68.4552) (end 81.6412 68.4552) (width 0.25) (layer F.Cu) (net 11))
 (segment (start 81.6412 68.4552) (end 78.5818 71.5146) (width 0.25) (layer F.Cu) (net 11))
 (segment (start 78.5818 71.5146) (end 78.5818 71.882) (width 0.25) (layer F.Cu) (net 11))
 (segment (start 77.4065 71.882) (end 78.5818 71.882) (width 0.25) (layer F.Cu) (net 11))
 (segment (start 129.984 72.136) (end 129.984 70.12) (width 0.25) (layer B.Cu) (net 11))
 (segment (start 129.984 70.12) (end 126.158 66.294) (width 0.25) (layer B.Cu) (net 11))
 (segment (start 124.908 63.794) (end 124.908 66.5967) (width 0.25) (layer F.Cu) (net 12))
 (segment (start 124.908 66.5967) (end 123.4998 68.0049) (width 0.25) (layer F.Cu) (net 12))
 (segment (start 123.4998 68.0049) (end 79.5516 68.0049) (width 0.25) (layer F.Cu) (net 12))
 (segment (start 79.5516 68.0049) (end 76.0418 71.5147) (width 0.25) (layer F.Cu) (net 12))
 (segment (start 76.0418 71.5147) (end 76.0418 71.882) (width 0.25) (layer F.Cu) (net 12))
 (segment (start 74.8665 71.882) (end 76.0418 71.882) (width 0.25) (layer F.Cu) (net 12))
 (segment (start 127.444 72.136) (end 127.444 69.4431) (width 0.25) (layer B.Cu) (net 12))
 (segment (start 127.444 69.4431) (end 124.908 66.9071) (width 0.25) (layer B.Cu) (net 12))
 (segment (start 124.908 66.9071) (end 124.908 63.794) (width 0.25) (layer B.Cu) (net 12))
 (segment (start 123.658 66.294) (end 122.3974 67.5546) (width 0.25) (layer F.Cu) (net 13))
 (segment (start 122.3974 67.5546) (end 77.4619 67.5546) (width 0.25) (layer F.Cu) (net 13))
 (segment (start 77.4619 67.5546) (end 73.5018 71.5147) (width 0.25) (layer F.Cu) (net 13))
 (segment (start 73.5018 71.5147) (end 73.5018 71.882) (width 0.25) (layer F.Cu) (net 13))
 (segment (start 72.3265 71.882) (end 73.5018 71.882) (width 0.25) (layer F.Cu) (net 13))
 (segment (start 124.904 72.136) (end 124.904 67.54) (width 0.25) (layer B.Cu) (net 13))
 (segment (start 124.904 67.54) (end 123.658 66.294) (width 0.25) (layer B.Cu) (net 13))
 (segment (start 64.7065 71.882) (end 65.8818 71.882) (width 0.25) (layer B.Cu) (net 14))
 (segment (start 117.284 72.136) (end 116.1087 72.136) (width 0.25) (layer B.Cu) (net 14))
 (segment (start 116.1087 72.136) (end 116.1087 72.5034) (width 0.25) (layer B.Cu) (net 14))
 (segment (start 116.1087 72.5034) (end 115.3008 73.3113) (width 0.25) (layer B.Cu) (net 14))
 (segment (start 115.3008 73.3113) (end 106.1379 73.3113) (width 0.25) (layer B.Cu) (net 14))
 (segment (start 106.1379 73.3113) (end 103.3505 76.0987) (width 0.25) (layer B.Cu) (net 14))
 (segment (start 103.3505 76.0987) (end 92.5956 76.0987) (width 0.25) (layer B.Cu) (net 14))
 (segment (start 92.5956 76.0987) (end 91.2819 74.785) (width 0.25) (layer B.Cu) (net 14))
 (segment (start 91.2819 74.785) (end 91.2819 73.8664) (width 0.25) (layer B.Cu) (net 14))
 (segment (start 91.2819 73.8664) (end 90.4728 73.0573) (width 0.25) (layer B.Cu) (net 14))
 (segment (start 90.4728 73.0573) (end 66.6897 73.0573) (width 0.25) (layer B.Cu) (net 14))
 (segment (start 66.6897 73.0573) (end 65.8818 72.2494) (width 0.25) (layer B.Cu) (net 14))
 (segment (start 65.8818 72.2494) (end 65.8818 71.882) (width 0.25) (layer B.Cu) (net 14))
 (segment (start 117.284 71.5483) (end 117.284 72.136) (width 0.25) (layer B.Cu) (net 14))
 (segment (start 117.284 70.9607) (end 121.158 67.0867) (width 0.25) (layer B.Cu) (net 14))
 (segment (start 121.158 67.0867) (end 121.158 66.294) (width 0.25) (layer B.Cu) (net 14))
 (segment (start 117.284 71.5483) (end 117.284 70.9607) (width 0.25) (layer B.Cu) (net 14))
 (segment (start 62.1665 71.882) (end 63.3418 71.882) (width 0.25) (layer F.Cu) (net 15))
 (segment (start 114.744 72.136) (end 113.5687 72.136) (width 0.25) (layer F.Cu) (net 15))
 (segment (start 113.5687 72.136) (end 113.5687 72.5033) (width 0.25) (layer F.Cu) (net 15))
 (segment (start 113.5687 72.5033) (end 112.7525 73.3195) (width 0.25) (layer F.Cu) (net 15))
 (segment (start 112.7525 73.3195) (end 106.6452 73.3195) (width 0.25) (layer F.Cu) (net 15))
 (segment (start 106.6452 73.3195) (end 106.383 73.0573) (width 0.25) (layer F.Cu) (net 15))
 (segment (start 106.383 73.0573) (end 64.1497 73.0573) (width 0.25) (layer F.Cu) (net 15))
 (segment (start 64.1497 73.0573) (end 63.3418 72.2494) (width 0.25) (layer F.Cu) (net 15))
 (segment (start 63.3418 72.2494) (end 63.3418 71.882) (width 0.25) (layer F.Cu) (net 15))
 (segment (start 114.744 70.9607) (end 115.552 70.9607) (width 0.25) (layer B.Cu) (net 15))
 (segment (start 115.552 70.9607) (end 119.908 66.6047) (width 0.25) (layer B.Cu) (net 15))
 (segment (start 119.908 66.6047) (end 119.908 63.794) (width 0.25) (layer B.Cu) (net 15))
 (segment (start 114.744 72.136) (end 114.744 70.9607) (width 0.25) (layer B.Cu) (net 15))
 (segment (start 99.822 63.881) (end 99.822 63.5994) (width 1.5) (layer F.Cu) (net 3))
 (segment (start 99.822 63.5994) (end 101.6161 61.8053) (width 1.5) (layer F.Cu) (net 3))
 (segment (start 101.6161 61.8053) (end 145.4193 61.8053) (width 1.5) (layer F.Cu) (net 3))
 (segment (start 145.4193 61.8053) (end 147.408 63.794) (width 1.5) (layer F.Cu) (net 3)))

